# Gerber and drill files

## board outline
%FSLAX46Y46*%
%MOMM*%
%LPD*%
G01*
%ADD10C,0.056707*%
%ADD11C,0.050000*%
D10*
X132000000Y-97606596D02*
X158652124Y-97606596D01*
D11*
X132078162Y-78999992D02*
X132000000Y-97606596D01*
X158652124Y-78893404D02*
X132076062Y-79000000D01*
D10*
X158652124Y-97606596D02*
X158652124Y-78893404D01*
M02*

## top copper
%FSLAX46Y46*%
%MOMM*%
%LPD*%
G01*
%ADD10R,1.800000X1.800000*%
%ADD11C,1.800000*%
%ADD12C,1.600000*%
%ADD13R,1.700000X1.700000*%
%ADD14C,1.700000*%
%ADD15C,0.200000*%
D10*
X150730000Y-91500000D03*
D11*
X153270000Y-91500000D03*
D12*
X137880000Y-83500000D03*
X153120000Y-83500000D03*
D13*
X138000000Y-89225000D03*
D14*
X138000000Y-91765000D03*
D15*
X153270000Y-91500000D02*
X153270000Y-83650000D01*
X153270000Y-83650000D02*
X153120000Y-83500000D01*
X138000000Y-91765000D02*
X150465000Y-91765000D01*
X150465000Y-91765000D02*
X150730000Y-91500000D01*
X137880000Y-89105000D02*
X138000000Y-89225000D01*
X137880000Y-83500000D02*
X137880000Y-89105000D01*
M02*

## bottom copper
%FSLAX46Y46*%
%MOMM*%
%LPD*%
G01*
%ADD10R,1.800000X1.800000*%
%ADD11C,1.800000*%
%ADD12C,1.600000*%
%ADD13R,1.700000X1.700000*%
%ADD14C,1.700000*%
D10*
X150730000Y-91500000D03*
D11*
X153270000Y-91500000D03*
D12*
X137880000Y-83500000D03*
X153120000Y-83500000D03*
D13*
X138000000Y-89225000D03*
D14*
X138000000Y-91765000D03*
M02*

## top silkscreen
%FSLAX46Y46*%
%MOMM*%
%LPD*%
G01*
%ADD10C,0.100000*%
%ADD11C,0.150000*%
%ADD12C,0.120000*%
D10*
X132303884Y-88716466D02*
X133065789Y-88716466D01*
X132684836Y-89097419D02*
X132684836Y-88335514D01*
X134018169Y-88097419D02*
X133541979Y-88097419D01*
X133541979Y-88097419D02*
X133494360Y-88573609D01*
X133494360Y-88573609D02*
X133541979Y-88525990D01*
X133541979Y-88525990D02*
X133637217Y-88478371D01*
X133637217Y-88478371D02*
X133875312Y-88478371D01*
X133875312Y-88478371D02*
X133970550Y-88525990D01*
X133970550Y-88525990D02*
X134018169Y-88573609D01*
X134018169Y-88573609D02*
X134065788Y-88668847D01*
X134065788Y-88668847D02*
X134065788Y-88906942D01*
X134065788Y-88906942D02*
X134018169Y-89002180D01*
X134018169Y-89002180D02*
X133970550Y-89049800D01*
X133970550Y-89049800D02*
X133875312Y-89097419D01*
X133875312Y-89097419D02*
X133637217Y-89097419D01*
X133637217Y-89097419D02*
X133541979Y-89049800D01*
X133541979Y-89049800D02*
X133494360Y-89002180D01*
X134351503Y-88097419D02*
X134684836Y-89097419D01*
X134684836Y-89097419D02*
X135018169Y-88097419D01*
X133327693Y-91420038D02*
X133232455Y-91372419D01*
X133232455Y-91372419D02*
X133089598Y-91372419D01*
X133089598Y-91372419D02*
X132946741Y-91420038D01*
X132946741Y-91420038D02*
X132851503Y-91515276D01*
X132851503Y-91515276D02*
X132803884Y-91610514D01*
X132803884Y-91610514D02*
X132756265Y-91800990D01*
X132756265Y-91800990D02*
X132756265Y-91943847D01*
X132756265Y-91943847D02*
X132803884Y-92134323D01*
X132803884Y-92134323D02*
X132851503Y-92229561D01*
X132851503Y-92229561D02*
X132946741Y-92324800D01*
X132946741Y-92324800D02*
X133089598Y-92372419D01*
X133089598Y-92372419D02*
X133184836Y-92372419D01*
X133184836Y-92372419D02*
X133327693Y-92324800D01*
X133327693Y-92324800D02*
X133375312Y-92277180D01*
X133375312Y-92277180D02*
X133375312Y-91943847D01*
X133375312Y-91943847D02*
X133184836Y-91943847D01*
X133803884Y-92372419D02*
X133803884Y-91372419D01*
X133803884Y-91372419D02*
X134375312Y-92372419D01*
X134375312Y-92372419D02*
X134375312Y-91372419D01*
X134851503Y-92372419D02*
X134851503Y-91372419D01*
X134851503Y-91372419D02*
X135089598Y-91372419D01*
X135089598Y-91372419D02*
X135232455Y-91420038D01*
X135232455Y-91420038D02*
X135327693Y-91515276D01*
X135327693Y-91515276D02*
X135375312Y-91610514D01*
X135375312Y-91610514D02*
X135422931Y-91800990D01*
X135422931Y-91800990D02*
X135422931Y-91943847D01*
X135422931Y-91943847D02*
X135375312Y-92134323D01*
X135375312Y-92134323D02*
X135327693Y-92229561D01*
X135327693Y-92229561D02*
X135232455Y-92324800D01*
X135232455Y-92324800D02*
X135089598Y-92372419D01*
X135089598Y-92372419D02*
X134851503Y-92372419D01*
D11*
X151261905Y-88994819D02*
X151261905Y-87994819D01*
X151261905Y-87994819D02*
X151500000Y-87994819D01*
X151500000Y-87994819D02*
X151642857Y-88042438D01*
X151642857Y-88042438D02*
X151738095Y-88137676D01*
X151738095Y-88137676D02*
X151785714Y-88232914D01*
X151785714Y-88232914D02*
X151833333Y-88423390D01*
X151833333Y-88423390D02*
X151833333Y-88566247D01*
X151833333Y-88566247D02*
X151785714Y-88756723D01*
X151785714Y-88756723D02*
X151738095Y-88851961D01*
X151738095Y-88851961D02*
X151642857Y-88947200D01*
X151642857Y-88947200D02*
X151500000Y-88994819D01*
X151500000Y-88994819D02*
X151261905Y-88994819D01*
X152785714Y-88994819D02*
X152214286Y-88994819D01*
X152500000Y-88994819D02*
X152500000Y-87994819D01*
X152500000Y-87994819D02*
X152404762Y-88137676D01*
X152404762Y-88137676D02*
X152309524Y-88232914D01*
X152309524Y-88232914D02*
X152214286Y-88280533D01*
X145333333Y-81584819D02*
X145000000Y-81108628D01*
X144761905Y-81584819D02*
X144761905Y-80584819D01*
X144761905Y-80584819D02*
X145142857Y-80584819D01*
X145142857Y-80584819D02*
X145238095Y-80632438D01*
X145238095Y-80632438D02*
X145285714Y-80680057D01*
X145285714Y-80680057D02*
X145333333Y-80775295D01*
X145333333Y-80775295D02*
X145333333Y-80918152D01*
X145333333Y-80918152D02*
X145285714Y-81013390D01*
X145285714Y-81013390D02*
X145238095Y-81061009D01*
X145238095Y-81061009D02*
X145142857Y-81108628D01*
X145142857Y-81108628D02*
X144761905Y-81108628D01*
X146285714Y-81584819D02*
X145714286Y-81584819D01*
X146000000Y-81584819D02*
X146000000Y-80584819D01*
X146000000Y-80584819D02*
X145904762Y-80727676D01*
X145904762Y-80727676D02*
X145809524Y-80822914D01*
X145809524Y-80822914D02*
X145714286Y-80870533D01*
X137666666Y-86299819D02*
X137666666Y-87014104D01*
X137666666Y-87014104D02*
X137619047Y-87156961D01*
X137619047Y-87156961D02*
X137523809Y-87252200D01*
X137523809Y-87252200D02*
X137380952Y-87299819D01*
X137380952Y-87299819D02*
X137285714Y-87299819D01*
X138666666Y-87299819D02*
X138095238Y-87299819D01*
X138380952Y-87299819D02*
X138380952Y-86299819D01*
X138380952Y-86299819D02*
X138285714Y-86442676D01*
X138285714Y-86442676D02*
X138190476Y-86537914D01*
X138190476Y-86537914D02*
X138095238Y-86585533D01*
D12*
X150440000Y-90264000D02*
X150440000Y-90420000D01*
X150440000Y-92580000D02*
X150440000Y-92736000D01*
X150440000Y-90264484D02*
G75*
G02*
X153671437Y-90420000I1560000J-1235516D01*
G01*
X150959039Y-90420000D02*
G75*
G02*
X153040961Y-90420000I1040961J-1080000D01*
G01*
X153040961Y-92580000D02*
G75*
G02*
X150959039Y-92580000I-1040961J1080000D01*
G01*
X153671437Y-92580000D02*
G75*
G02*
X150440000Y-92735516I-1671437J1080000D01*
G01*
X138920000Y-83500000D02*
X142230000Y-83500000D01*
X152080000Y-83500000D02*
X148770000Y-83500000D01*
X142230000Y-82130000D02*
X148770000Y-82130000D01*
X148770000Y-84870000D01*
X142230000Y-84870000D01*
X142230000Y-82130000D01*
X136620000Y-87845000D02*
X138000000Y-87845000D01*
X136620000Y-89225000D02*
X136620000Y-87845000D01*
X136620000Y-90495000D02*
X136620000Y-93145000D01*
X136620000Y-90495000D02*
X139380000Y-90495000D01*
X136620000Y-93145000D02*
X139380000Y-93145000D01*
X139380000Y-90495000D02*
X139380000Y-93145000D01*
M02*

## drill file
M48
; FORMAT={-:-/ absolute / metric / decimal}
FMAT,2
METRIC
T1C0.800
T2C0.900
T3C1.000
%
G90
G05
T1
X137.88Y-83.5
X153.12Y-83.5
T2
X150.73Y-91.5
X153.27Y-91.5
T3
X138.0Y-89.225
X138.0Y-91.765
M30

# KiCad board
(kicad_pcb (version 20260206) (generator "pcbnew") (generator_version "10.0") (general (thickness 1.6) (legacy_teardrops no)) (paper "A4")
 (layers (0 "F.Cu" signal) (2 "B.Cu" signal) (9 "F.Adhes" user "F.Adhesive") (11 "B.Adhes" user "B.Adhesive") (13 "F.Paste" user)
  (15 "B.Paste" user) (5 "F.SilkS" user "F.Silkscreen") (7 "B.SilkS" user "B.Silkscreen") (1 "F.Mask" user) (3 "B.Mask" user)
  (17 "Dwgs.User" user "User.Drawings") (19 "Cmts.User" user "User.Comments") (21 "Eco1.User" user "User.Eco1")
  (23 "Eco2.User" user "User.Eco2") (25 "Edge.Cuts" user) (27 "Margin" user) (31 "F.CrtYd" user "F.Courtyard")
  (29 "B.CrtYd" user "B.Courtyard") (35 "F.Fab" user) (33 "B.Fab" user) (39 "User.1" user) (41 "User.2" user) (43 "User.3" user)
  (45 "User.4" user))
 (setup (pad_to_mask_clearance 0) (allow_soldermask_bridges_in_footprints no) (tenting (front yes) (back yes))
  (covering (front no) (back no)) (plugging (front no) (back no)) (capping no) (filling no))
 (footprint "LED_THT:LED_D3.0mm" (layer "F.Cu") (at 150.73 91.5)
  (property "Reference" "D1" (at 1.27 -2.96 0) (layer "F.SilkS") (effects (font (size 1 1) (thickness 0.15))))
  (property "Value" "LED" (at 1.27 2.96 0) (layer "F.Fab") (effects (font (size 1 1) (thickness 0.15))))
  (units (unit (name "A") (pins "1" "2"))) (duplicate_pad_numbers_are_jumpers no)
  (fp_line (start -0.29 -1.236) (end -0.29 -1.08) (stroke (width 0.12) (type solid)) (layer "F.SilkS"))
  (fp_line (start -0.29 1.08) (end -0.29 1.236) (stroke (width 0.12) (type solid)) (layer "F.SilkS"))
  (fp_arc (start -0.29 -1.235516) (mid 1.36566 -1.987699) (end 2.941437 -1.08) (stroke (width 0.12) (type solid)) (layer "F.SilkS"))
  (fp_arc (start 0.229039 -1.08) (mid 1.27 -1.5) (end 2.310961 -1.08) (stroke (width 0.12) (type solid)) (layer "F.SilkS"))
  (fp_arc (start 2.310961 1.08) (mid 1.27 1.5) (end 0.229039 1.08) (stroke (width 0.12) (type solid)) (layer "F.SilkS"))
  (fp_arc (start 2.941437 1.08) (mid 1.36566 1.987699) (end -0.29 1.235516) (stroke (width 0.12) (type solid)) (layer "F.SilkS"))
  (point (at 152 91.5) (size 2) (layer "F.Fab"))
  (pad "1" thru_hole rect (at 0 0) (size 1.8 1.8) (drill 0.9) (layers "*.Cu" "*.Mask") (remove_unused_layers no) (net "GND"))
  (pad "2" thru_hole circle (at 2.54 0) (size 1.8 1.8) (drill 0.9) (layers "*.Cu" "*.Mask") (remove_unused_layers no) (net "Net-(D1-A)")))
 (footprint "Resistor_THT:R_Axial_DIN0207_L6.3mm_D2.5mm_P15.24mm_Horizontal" (layer "F.Cu") (at 137.88 83.5)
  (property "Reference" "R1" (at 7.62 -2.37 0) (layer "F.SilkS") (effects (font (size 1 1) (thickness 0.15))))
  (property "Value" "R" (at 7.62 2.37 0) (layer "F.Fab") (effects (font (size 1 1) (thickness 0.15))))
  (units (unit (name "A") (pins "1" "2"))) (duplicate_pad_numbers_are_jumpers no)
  (fp_line (start 1.04 0) (end 4.35 0) (stroke (width 0.12) (type solid)) (layer "F.SilkS"))
  (fp_line (start 14.2 0) (end 10.89 0) (stroke (width 0.12) (type solid)) (layer "F.SilkS"))
  (fp_rect (start 4.35 -1.37) (end 10.89 1.37) (stroke (width 0.12) (type solid)) (fill no) (layer "F.SilkS"))
  (pad "1" thru_hole circle (at 0 0) (size 1.6 1.6) (drill 0.8) (layers "*.Cu" "*.Mask") (remove_unused_layers no) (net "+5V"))
  (pad "2" thru_hole circle (at 15.24 0) (size 1.6 1.6) (drill 0.8) (layers "*.Cu" "*.Mask") (remove_unused_layers no) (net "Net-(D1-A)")))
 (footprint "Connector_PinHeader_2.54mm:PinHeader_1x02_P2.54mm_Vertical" (layer "F.Cu") (at 138 89.225)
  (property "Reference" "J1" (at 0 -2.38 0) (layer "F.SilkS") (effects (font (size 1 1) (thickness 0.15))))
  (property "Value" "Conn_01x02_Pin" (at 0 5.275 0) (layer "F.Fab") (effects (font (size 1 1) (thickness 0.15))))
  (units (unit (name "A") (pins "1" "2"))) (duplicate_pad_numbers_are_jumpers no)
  (fp_line (start -1.38 -1.38) (end 0 -1.38) (stroke (width 0.12) (type solid)) (layer "F.SilkS"))
  (fp_line (start -1.38 0) (end -1.38 -1.38) (stroke (width 0.12) (type solid)) (layer "F.SilkS"))
  (fp_line (start -1.38 1.27) (end -1.38 3.92) (stroke (width 0.12) (type solid)) (layer "F.SilkS"))
  (fp_line (start -1.38 1.27) (end 1.38 1.27) (stroke (width 0.12) (type solid)) (layer "F.SilkS"))
  (fp_line (start -1.38 3.92) (end 1.38 3.92) (stroke (width 0.12) (type solid)) (layer "F.SilkS"))
  (fp_line (start 1.38 1.27) (end 1.38 3.92) (stroke (width 0.12) (type solid)) (layer "F.SilkS"))
  (pad "1" thru_hole rect (at 0 0) (size 1.7 1.7) (drill 1) (layers "*.Cu" "*.Mask") (remove_unused_layers no) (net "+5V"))
  (pad "2" thru_hole circle (at 0 2.54) (size 1.7 1.7) (drill 1) (layers "*.Cu" "*.Mask") (remove_unused_layers no) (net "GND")))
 (gr_line (start 132 97.606596) (end 158.652124 97.606596) (stroke (width 0.056707) (type default)) (layer "Edge.Cuts"))
 (gr_line (start 132.078162 78.999992) (end 132 97.606596) (stroke (width 0.05) (type default)) (layer "Edge.Cuts"))
 (gr_line (start 158.652124 78.893404) (end 132.076062 79) (stroke (width 0.05) (type default)) (layer "Edge.Cuts"))
 (gr_line (start 158.652124 97.606596) (end 158.652124 78.893404) (stroke (width 0.056707) (type default)) (layer "Edge.Cuts"))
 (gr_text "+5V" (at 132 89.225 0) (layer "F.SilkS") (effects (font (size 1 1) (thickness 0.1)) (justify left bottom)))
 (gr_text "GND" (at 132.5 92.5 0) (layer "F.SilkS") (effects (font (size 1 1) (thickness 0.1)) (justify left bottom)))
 (segment (start 153.27 91.5) (end 153.27 83.65) (width 0.2) (layer "F.Cu") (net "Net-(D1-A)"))
 (segment (start 153.27 83.65) (end 153.12 83.5) (width 0.2) (layer "F.Cu") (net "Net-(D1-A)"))
 (segment (start 138 91.765) (end 150.465 91.765) (width 0.2) (layer "F.Cu") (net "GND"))
 (segment (start 150.465 91.765) (end 150.73 91.5) (width 0.2) (layer "F.Cu") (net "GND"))
 (segment (start 137.88 89.105) (end 138 89.225) (width 0.2) (layer "F.Cu") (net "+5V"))
 (segment (start 137.88 83.5) (end 137.88 89.105) (width 0.2) (layer "F.Cu") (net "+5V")))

